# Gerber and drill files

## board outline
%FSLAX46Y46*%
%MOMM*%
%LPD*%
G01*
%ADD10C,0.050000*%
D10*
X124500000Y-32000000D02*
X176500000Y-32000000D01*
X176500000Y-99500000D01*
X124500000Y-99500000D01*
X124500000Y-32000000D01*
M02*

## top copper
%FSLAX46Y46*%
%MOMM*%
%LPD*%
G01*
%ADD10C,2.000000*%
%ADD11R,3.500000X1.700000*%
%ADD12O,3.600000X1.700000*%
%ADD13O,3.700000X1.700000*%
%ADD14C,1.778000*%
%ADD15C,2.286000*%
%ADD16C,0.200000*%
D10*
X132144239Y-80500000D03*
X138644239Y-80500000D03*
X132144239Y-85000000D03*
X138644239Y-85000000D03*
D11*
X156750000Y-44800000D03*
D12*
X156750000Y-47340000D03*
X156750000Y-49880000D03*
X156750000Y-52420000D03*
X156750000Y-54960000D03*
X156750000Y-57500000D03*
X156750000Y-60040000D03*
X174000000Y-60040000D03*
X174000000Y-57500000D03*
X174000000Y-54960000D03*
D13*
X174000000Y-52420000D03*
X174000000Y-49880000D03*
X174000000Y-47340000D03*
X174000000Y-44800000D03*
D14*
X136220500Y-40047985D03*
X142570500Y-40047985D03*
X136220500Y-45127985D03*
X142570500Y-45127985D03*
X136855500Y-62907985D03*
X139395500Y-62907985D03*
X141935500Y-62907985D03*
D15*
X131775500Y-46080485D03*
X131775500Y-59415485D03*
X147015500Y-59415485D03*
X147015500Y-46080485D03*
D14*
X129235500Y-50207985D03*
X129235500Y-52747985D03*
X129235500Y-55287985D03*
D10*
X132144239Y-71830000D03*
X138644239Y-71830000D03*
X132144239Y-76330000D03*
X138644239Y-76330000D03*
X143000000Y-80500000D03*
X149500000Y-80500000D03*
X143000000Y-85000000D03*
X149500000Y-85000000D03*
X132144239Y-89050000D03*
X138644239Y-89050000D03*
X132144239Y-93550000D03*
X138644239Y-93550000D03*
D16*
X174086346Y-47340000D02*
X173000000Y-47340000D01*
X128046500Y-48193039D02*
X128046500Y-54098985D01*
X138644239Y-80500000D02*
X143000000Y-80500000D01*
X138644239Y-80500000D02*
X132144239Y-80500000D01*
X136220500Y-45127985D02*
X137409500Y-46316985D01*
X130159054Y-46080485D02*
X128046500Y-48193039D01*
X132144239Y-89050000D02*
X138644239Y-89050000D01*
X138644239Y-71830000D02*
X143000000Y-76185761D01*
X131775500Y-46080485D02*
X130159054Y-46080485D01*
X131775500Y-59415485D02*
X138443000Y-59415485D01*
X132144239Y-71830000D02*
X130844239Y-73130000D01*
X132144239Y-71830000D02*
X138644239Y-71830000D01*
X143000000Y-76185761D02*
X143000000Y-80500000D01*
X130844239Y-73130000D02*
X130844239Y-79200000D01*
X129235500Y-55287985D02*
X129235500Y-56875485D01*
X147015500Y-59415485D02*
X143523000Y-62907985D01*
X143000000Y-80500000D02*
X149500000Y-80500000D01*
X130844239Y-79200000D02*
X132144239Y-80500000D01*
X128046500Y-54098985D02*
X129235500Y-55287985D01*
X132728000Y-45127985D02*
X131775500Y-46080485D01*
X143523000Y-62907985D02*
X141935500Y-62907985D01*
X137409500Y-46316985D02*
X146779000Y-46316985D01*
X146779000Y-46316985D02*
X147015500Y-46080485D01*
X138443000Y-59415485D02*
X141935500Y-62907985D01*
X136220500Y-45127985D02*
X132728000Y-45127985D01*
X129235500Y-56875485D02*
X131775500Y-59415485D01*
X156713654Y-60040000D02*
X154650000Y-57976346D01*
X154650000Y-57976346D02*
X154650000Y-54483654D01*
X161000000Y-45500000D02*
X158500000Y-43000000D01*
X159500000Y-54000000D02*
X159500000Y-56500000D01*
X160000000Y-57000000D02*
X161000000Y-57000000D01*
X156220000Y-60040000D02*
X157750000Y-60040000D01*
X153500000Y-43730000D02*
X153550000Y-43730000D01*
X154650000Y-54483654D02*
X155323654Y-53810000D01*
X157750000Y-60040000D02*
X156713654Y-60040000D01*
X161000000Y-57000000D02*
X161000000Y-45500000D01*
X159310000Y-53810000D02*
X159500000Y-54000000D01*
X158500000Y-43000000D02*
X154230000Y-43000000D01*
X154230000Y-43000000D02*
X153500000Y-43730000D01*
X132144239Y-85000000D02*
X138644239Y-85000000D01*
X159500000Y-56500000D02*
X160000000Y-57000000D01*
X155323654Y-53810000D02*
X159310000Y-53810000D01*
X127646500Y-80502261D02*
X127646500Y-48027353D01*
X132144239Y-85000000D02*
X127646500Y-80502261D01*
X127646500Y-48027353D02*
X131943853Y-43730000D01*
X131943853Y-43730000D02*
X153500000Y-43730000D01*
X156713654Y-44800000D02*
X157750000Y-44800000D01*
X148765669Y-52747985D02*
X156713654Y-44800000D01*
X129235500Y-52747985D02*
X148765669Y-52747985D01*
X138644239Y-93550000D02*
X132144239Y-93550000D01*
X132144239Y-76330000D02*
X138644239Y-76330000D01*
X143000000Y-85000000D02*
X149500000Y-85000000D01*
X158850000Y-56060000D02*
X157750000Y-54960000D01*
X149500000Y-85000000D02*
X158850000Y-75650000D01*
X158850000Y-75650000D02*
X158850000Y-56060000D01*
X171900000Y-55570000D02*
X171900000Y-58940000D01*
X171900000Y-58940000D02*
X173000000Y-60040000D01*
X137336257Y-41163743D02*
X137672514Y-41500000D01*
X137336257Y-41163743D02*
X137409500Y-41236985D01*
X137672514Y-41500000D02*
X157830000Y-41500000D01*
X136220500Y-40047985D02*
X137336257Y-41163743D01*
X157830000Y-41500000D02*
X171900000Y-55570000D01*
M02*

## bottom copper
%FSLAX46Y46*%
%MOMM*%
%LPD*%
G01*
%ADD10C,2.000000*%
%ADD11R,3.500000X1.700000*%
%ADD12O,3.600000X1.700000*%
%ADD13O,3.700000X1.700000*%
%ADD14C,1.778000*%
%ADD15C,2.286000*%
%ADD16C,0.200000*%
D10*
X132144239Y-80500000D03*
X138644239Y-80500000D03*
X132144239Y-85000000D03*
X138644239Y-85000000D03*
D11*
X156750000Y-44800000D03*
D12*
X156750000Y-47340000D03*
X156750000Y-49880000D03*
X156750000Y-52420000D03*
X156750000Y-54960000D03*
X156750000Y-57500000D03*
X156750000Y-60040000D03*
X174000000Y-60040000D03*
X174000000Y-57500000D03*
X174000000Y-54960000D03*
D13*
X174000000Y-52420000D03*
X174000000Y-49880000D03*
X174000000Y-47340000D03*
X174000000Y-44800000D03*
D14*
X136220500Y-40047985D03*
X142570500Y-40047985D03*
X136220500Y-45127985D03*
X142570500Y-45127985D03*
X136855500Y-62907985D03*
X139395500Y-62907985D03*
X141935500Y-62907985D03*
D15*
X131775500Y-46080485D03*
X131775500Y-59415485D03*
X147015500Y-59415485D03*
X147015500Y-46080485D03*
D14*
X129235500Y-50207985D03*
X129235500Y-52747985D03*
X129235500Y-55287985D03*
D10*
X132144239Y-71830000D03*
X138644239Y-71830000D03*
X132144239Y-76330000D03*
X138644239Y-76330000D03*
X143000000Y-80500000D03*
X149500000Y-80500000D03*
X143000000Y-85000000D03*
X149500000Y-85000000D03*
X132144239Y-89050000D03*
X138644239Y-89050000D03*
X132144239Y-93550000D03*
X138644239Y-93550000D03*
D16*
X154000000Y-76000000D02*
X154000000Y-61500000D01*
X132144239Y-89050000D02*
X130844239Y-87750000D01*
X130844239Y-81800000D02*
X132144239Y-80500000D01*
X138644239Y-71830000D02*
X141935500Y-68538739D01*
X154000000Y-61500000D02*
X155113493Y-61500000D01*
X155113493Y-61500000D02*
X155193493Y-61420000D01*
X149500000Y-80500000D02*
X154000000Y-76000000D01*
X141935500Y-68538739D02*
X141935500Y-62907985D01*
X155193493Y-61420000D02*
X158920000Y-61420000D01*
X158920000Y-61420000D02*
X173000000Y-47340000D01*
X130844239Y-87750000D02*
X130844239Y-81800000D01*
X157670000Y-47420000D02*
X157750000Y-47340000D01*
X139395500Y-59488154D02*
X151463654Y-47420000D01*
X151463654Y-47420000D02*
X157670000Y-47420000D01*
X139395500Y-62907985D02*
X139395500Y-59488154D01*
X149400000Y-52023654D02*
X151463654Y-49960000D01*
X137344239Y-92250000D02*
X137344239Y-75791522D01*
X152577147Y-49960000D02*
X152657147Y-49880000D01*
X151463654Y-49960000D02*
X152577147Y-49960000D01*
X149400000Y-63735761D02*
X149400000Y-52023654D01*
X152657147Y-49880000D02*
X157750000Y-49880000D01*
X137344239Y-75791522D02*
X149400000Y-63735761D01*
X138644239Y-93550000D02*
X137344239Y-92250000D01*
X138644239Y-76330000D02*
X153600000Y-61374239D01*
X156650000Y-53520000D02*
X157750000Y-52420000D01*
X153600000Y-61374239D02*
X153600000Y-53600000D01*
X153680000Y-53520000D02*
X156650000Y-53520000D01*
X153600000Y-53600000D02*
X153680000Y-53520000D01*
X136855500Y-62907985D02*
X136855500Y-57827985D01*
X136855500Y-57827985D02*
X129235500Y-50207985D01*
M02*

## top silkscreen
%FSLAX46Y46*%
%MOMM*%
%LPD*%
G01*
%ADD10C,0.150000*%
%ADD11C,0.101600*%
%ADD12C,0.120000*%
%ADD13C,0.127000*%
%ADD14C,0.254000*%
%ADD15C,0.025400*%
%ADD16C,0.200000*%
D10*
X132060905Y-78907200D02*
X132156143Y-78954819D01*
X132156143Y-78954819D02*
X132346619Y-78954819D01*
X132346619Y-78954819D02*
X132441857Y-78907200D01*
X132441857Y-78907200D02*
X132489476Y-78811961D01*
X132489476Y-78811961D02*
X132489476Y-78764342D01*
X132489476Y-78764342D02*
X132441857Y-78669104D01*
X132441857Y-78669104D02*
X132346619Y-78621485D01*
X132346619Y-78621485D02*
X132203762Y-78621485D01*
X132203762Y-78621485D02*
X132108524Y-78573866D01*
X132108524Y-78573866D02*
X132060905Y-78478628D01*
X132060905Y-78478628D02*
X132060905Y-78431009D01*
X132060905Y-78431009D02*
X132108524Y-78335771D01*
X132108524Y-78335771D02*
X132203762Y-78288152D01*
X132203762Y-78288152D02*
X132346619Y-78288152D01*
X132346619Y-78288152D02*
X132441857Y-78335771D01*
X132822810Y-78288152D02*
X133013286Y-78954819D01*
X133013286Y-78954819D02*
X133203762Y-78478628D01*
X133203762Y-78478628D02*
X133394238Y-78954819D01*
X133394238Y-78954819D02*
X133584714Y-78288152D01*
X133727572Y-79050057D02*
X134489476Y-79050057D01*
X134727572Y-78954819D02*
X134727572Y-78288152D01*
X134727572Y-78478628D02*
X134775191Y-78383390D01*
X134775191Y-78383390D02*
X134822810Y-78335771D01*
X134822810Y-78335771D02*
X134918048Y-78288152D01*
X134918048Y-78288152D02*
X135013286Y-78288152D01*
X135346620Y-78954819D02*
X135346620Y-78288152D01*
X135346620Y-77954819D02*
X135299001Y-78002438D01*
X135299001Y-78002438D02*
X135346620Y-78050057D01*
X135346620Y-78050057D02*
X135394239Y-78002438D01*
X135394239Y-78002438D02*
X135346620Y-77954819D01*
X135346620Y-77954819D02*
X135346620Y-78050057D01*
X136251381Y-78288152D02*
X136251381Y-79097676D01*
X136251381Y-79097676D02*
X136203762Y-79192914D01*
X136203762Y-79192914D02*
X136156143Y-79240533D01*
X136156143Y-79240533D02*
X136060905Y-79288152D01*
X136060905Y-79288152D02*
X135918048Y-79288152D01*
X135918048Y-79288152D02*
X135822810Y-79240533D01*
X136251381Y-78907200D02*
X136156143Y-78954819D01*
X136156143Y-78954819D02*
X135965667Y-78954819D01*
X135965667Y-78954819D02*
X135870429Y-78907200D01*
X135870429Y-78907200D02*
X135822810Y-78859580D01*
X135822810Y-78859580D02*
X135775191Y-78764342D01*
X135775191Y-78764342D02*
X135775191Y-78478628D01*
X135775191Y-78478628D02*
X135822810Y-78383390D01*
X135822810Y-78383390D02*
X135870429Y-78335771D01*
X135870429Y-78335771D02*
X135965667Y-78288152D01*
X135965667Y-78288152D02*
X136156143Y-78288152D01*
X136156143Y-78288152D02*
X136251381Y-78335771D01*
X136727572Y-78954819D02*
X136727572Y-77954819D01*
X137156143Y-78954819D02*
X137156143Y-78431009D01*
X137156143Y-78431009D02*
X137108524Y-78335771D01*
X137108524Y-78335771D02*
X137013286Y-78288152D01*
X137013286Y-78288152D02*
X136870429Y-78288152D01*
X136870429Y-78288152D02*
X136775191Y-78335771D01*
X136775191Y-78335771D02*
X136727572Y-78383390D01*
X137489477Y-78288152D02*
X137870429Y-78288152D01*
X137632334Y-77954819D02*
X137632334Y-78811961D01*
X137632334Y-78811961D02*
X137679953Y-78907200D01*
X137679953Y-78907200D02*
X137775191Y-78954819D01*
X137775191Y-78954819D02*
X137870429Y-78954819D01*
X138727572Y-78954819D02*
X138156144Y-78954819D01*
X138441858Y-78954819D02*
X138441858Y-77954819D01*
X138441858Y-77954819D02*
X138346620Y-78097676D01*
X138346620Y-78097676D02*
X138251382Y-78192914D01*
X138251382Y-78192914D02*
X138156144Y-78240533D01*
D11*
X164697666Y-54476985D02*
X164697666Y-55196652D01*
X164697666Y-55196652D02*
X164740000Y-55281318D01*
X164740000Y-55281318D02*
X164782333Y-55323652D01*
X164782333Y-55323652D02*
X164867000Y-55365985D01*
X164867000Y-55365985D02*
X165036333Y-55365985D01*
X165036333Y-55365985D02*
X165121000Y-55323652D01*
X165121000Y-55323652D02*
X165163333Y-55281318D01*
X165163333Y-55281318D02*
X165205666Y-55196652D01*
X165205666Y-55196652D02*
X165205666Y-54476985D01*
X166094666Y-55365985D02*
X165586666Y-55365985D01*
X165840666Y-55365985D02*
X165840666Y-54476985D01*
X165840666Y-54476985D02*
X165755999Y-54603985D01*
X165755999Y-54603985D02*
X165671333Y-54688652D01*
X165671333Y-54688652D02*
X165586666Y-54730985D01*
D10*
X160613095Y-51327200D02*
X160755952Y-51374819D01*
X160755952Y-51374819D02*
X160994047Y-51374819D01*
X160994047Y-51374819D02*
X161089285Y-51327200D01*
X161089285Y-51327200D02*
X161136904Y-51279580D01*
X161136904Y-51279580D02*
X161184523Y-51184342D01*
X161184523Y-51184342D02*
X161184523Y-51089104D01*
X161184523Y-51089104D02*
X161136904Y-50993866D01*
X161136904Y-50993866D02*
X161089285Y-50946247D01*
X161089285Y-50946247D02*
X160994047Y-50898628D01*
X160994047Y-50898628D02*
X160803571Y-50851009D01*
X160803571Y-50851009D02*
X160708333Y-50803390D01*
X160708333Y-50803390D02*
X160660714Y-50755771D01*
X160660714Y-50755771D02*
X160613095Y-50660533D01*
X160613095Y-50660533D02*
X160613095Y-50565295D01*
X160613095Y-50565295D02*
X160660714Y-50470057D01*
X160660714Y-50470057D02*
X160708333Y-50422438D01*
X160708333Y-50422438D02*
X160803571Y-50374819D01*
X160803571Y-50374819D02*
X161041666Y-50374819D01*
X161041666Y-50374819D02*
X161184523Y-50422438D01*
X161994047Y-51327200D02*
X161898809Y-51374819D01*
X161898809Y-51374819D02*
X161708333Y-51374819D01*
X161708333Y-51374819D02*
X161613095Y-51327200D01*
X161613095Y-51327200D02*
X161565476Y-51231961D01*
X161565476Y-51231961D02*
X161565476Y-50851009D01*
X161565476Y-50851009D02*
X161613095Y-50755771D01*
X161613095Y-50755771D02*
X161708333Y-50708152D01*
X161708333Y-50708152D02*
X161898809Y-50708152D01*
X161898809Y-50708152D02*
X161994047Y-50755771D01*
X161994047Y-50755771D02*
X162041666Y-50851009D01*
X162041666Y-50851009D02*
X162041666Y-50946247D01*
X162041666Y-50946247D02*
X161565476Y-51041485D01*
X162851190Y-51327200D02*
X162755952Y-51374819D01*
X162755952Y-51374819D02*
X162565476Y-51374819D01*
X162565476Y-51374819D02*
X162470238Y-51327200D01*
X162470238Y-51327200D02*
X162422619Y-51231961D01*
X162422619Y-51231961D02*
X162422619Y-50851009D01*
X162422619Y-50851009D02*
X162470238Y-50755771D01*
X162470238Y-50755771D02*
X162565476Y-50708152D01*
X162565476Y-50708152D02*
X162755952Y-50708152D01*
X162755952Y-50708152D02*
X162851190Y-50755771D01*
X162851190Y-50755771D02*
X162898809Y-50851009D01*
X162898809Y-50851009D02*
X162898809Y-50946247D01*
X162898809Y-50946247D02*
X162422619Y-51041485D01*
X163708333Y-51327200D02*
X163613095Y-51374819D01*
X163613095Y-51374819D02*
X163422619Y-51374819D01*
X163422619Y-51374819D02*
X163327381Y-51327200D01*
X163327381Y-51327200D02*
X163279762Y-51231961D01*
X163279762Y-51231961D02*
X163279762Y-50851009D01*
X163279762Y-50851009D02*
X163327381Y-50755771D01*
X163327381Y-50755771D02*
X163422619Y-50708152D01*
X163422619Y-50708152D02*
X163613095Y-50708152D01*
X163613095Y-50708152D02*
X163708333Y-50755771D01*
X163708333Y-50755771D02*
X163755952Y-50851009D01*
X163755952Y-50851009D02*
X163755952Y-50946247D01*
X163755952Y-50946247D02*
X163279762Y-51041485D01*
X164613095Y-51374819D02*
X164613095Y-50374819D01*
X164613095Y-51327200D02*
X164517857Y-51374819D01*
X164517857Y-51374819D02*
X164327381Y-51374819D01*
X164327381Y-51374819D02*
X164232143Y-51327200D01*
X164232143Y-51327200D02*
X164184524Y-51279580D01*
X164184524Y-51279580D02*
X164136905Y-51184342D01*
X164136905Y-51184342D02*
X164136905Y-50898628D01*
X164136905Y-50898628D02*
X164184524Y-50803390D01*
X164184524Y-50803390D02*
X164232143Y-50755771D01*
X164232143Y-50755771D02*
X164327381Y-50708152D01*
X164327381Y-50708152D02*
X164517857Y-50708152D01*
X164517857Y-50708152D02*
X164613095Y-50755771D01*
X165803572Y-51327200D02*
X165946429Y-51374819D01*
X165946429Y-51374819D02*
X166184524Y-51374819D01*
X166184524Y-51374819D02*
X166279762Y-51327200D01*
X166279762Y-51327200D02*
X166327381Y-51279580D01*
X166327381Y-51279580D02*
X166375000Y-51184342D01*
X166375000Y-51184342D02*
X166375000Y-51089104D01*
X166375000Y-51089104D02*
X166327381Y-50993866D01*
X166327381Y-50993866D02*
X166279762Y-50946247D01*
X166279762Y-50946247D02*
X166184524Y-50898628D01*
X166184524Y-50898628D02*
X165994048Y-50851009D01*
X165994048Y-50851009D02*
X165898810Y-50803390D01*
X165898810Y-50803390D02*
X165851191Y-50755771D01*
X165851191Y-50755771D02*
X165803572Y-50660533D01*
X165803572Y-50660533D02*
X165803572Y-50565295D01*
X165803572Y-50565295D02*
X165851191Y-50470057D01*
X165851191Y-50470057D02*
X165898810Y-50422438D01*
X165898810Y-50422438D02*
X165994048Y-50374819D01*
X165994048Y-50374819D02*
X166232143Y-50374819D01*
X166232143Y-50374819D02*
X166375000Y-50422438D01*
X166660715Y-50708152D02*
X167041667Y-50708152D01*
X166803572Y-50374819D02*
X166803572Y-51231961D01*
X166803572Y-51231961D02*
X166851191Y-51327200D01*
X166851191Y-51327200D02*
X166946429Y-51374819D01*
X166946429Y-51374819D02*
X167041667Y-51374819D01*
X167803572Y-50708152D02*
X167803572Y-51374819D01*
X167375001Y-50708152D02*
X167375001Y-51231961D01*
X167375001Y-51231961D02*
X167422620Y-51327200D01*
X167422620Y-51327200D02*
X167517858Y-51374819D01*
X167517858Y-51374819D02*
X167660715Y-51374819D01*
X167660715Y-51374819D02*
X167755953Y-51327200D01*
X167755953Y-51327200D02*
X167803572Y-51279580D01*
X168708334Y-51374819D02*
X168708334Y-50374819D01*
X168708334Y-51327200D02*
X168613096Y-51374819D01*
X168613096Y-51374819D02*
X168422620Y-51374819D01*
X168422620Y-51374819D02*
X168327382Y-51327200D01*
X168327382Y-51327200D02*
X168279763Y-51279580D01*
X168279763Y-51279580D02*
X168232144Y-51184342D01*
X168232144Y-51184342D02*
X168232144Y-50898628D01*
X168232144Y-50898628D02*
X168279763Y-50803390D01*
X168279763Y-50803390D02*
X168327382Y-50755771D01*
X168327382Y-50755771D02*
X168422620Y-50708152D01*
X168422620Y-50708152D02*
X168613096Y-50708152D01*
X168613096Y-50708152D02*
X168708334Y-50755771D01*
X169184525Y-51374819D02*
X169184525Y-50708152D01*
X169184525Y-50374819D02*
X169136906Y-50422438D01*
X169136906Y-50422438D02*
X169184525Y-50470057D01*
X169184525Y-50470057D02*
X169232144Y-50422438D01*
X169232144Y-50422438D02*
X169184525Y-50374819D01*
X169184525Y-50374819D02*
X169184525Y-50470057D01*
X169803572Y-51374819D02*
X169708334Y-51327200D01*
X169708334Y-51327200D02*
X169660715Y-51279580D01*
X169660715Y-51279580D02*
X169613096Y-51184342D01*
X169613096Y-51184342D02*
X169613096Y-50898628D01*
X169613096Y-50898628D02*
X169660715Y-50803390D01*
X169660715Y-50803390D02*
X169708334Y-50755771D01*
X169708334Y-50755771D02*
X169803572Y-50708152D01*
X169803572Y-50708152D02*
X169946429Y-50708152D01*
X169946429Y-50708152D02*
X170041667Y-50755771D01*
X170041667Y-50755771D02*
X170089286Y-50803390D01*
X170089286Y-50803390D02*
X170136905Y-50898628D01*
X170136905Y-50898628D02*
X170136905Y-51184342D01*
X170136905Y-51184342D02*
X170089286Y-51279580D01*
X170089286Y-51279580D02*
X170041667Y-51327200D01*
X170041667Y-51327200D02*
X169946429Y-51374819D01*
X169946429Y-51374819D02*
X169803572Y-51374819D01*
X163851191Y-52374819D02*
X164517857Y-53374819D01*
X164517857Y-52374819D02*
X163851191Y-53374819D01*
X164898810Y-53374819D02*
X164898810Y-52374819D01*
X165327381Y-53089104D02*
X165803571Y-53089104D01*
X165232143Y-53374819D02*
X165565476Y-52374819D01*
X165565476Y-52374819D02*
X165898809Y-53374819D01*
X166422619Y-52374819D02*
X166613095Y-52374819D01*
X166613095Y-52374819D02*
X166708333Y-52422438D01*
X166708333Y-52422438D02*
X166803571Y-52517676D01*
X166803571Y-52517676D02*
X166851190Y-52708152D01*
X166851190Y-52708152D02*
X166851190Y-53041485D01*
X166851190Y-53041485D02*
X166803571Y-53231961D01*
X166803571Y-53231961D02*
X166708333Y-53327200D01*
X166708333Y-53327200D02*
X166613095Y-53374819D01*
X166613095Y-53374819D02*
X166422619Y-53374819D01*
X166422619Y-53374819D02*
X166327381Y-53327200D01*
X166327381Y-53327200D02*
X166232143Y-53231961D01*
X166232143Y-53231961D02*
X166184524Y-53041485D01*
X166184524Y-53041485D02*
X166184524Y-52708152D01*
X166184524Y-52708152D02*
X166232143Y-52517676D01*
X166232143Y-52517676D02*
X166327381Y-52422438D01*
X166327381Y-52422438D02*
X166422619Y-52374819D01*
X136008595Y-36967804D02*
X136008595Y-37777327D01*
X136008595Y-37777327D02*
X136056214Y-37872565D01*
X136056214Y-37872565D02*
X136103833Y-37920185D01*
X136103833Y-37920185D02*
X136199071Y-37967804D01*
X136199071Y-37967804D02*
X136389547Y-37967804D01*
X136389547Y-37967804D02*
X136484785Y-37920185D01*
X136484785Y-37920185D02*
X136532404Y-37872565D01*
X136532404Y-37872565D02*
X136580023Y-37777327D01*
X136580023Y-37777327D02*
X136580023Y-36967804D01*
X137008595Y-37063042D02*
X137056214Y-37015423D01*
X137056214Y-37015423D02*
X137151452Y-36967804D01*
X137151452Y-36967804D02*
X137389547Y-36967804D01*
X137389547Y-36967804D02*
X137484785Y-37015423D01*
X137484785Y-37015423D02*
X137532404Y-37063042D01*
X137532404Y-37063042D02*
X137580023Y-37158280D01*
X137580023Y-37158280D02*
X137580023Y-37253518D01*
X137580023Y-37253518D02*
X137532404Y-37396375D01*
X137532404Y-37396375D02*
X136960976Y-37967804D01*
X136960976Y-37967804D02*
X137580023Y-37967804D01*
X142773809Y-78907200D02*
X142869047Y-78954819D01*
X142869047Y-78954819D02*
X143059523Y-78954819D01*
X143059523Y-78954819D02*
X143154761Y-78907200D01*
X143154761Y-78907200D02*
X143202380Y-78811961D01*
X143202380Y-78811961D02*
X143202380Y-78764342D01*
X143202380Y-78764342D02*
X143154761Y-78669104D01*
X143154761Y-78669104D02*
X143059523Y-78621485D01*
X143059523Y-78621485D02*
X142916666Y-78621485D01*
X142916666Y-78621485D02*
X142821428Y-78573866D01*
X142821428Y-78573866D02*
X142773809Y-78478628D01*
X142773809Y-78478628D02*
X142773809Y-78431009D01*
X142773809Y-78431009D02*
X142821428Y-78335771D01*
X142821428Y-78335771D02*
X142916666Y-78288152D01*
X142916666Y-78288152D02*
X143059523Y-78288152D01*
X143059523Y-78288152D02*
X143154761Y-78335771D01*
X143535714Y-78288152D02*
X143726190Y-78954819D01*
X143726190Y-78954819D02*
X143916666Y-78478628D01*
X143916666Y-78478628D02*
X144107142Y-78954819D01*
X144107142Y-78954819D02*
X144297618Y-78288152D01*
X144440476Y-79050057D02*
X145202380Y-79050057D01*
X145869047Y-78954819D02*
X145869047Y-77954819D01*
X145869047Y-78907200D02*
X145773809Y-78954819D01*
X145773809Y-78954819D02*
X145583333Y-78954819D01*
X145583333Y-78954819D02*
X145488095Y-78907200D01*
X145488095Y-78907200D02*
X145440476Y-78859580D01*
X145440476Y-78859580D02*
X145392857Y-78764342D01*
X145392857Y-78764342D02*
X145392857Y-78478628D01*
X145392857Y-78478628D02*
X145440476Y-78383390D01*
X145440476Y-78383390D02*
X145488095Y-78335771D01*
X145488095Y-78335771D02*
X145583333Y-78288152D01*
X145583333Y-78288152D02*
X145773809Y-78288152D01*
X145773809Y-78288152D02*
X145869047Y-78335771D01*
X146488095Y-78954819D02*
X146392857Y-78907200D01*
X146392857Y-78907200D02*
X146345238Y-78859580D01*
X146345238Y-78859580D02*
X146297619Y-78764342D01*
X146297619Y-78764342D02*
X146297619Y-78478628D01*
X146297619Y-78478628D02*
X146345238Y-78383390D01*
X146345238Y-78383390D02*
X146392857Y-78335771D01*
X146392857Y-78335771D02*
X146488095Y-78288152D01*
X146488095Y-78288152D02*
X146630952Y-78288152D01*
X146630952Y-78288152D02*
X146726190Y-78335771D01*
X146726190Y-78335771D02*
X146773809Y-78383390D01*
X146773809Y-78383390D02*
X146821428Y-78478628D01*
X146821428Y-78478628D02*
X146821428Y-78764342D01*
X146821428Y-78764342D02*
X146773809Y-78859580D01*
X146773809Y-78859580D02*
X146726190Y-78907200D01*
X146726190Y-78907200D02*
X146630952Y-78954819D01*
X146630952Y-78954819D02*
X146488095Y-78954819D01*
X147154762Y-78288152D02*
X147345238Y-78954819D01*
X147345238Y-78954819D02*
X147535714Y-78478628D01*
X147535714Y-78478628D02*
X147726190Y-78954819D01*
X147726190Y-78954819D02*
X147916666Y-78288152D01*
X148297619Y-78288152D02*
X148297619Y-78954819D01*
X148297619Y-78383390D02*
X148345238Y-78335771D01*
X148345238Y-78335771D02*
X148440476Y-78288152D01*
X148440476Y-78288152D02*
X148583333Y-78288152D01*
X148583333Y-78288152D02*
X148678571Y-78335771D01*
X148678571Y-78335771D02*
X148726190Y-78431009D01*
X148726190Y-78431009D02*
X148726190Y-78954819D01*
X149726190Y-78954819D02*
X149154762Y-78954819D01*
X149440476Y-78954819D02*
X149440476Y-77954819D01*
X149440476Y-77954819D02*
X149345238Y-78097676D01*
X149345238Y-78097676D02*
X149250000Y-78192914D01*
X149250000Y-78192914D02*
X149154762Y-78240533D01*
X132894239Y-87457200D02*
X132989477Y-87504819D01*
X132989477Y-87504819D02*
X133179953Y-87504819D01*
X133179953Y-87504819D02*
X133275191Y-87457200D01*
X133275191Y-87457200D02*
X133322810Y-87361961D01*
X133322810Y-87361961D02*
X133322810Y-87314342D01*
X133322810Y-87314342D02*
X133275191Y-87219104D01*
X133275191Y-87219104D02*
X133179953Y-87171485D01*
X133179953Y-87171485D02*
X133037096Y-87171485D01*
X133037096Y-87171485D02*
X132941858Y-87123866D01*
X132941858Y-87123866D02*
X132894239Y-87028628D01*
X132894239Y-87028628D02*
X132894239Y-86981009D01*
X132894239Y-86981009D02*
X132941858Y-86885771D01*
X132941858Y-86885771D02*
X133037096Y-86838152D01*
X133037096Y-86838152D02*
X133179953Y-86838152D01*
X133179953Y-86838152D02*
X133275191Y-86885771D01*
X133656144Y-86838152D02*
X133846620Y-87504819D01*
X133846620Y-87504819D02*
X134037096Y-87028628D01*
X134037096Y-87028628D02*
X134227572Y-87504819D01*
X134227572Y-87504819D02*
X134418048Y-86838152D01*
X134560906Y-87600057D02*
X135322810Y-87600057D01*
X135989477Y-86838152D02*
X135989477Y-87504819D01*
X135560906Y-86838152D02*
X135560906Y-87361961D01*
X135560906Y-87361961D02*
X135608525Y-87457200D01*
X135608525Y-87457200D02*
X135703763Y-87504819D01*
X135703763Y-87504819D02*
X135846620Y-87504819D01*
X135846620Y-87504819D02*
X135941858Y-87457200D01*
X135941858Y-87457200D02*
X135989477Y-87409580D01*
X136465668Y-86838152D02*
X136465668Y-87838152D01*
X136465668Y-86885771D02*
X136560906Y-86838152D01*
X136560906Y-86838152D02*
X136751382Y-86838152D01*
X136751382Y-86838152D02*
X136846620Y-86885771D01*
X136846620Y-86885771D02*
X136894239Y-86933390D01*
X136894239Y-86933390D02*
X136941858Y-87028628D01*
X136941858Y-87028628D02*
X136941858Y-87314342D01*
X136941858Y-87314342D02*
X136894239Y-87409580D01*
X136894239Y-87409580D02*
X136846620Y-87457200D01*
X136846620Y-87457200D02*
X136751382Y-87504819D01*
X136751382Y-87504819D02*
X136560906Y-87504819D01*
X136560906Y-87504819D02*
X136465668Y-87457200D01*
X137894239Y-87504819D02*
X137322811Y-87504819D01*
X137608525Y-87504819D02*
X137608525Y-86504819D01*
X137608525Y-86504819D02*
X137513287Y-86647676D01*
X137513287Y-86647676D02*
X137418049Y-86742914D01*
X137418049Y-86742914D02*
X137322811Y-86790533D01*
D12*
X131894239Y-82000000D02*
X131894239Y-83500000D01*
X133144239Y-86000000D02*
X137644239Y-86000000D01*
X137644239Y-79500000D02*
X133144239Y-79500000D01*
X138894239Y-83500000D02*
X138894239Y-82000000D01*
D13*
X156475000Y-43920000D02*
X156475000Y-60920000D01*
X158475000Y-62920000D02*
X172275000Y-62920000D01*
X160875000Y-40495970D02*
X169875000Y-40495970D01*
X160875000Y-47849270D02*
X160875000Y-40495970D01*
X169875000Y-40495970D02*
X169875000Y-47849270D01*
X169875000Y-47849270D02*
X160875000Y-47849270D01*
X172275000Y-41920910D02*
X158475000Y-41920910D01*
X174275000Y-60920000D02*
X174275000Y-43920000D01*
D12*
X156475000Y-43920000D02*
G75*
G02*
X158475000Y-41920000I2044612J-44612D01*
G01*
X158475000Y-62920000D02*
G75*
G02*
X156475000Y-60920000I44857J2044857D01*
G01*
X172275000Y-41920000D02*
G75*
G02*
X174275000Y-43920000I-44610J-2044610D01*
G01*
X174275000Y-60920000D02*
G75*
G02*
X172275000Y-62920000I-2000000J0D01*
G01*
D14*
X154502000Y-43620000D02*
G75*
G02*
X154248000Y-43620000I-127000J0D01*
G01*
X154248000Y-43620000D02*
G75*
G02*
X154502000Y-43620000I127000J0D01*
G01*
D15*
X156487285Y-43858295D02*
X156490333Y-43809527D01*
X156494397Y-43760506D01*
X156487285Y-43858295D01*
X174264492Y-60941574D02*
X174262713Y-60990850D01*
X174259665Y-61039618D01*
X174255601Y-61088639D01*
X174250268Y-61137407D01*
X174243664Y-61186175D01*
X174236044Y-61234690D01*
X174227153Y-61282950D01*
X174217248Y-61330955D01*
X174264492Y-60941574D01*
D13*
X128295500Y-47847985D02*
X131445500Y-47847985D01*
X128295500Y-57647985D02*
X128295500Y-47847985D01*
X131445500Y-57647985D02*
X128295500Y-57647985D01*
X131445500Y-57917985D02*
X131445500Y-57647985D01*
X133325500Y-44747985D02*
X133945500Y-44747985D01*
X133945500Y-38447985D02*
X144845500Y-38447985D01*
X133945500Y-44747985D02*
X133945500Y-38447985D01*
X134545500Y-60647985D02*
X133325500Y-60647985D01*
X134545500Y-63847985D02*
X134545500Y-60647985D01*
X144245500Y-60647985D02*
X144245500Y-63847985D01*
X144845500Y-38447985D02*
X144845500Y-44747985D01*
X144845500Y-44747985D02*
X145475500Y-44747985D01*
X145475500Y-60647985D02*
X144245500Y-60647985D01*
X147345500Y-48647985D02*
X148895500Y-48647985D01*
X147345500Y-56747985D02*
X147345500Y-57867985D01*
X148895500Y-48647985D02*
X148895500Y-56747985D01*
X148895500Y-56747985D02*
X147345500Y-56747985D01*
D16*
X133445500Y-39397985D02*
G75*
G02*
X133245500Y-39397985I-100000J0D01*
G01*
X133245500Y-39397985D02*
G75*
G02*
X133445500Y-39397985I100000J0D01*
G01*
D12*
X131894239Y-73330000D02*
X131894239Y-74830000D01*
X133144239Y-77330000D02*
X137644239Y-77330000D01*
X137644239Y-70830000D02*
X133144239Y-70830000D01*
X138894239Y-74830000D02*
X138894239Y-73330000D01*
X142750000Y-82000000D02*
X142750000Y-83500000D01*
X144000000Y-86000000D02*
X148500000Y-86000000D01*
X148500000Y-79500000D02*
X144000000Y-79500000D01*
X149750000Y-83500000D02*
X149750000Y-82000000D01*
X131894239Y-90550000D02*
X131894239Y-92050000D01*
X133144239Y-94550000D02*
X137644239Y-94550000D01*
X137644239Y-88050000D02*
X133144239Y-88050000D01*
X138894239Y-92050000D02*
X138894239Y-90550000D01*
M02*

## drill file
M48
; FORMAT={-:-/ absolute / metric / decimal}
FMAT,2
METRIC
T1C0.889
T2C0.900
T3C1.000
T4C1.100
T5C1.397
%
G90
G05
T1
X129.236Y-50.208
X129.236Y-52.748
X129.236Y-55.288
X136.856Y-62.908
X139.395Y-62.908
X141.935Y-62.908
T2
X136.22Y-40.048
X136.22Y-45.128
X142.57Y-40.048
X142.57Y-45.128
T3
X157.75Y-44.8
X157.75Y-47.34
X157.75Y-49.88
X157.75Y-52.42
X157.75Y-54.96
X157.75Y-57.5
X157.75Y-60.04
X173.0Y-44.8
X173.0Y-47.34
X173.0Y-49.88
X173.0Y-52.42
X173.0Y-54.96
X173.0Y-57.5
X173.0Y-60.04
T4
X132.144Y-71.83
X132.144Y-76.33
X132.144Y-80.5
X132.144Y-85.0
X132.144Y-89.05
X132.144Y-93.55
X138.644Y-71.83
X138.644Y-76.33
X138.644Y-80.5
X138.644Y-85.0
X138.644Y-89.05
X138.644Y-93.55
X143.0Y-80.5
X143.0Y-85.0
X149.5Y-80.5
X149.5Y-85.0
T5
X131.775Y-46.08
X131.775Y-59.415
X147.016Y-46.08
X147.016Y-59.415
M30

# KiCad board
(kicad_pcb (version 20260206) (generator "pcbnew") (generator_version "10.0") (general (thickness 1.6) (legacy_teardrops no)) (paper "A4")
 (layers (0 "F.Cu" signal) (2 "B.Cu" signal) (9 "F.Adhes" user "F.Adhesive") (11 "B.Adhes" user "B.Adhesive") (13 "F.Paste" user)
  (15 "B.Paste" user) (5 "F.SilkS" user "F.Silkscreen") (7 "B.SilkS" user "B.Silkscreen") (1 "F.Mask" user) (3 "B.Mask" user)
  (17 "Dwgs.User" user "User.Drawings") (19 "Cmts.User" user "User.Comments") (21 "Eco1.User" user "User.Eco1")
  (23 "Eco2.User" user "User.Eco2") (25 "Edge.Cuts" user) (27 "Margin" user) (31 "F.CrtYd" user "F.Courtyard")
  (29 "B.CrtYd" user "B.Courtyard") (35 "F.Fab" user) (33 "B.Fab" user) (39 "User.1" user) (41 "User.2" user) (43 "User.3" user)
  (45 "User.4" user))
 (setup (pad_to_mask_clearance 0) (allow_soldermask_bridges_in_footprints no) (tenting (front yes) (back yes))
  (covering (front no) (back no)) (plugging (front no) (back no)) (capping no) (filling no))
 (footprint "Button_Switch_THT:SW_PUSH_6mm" (layer "F.Cu") (at 132.144239 80.5)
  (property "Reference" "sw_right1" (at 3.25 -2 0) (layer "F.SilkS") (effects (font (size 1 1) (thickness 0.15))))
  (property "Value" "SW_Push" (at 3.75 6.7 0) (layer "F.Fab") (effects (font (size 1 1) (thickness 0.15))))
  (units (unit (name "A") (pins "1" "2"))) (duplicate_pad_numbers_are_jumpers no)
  (fp_line (start -0.25 1.5) (end -0.25 3) (stroke (width 0.12) (type solid)) (layer "F.SilkS"))
  (fp_line (start 1 5.5) (end 5.5 5.5) (stroke (width 0.12) (type solid)) (layer "F.SilkS"))
  (fp_line (start 5.5 -1) (end 1 -1) (stroke (width 0.12) (type solid)) (layer "F.SilkS"))
  (fp_line (start 6.75 3) (end 6.75 1.5) (stroke (width 0.12) (type solid)) (layer "F.SilkS"))
  (pad "1" thru_hole circle (at 0 0 90) (size 2 2) (drill 1.1) (layers "*.Cu" "*.Mask") (remove_unused_layers no) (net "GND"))
  (pad "1" thru_hole circle (at 6.5 0 90) (size 2 2) (drill 1.1) (layers "*.Cu" "*.Mask") (remove_unused_layers no) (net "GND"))
  (pad "2" thru_hole circle (at 0 4.5 90) (size 2 2) (drill 1.1) (layers "*.Cu" "*.Mask") (remove_unused_layers no)
   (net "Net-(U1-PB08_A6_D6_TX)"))
  (pad "2" thru_hole circle (at 6.5 4.5 90) (size 2 2) (drill 1.1) (layers "*.Cu" "*.Mask") (remove_unused_layers no)
   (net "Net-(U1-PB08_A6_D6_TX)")))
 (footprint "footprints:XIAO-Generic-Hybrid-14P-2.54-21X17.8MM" (layer "F.Cu") (at 165.375 52.42)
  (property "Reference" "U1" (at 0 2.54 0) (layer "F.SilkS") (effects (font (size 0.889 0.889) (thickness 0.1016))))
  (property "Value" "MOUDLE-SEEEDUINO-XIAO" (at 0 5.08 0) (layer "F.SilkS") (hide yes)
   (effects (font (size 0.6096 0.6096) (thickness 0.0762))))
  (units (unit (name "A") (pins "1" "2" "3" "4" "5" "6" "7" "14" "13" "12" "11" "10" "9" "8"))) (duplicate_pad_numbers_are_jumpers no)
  (fp_line (start -8.9 -8.5) (end -8.9 8.5) (stroke (width 0.127) (type solid)) (layer "F.SilkS"))
  (fp_line (start -6.9 10.5) (end 6.9 10.5) (stroke (width 0.127) (type solid)) (layer "F.SilkS"))
  (fp_line (start -4.5 -11.92403) (end 4.5 -11.92403) (stroke (width 0.127) (type solid)) (layer "F.SilkS"))
  (fp_line (start -4.5 -4.57073) (end -4.5 -11.92403) (stroke (width 0.127) (type solid)) (layer "F.SilkS"))
  (fp_line (start 4.5 -11.92403) (end 4.5 -4.57073) (stroke (width 0.127) (type solid)) (layer "F.SilkS"))
  (fp_line (start 4.5 -4.57073) (end -4.5 -4.57073) (stroke (width 0.127) (type solid)) (layer "F.SilkS"))
  (fp_line (start 6.9 -10.49909) (end -6.9 -10.49909) (stroke (width 0.127) (type solid)) (layer "F.SilkS"))
  (fp_line (start 8.9 8.5) (end 8.9 -8.5) (stroke (width 0.127) (type solid)) (layer "F.SilkS"))
  (fp_arc (start -8.9 -8.5) (mid -8.301491 -9.901491) (end -6.9 -10.5) (stroke (width 0.12) (type solid)) (layer "F.SilkS"))
  (fp_arc (start -6.9 10.5) (mid -8.301423 9.901423) (end -8.9 8.5) (stroke (width 0.12) (type solid)) (layer "F.SilkS"))
  (fp_arc (start 6.9 -10.5) (mid 8.301491 -9.901491) (end 8.9 -8.5) (stroke (width 0.12) (type solid)) (layer "F.SilkS"))
  (fp_arc (start 8.9 8.5) (mid 8.314214 9.914214) (end 6.9 10.5) (stroke (width 0.12) (type solid)) (layer "F.SilkS"))
  (fp_circle (center -11 -8.8) (end -11 -9.054) (stroke (width 0) (type solid)) (fill yes) (layer "F.SilkS"))
  (fp_poly
   (pts (xy -8.887715 -8.561705) (xy -8.884667 -8.610473) (xy -8.880603 -8.659494)) (stroke (width 0.0254) (type solid)) (fill no)
   (layer "F.SilkS"))
  (fp_poly
   (pts (xy 8.889492 8.521574) (xy 8.887713 8.57085) (xy 8.884665 8.619618) (xy 8.880601 8.668639) (xy 8.875268 8.717407)
    (xy 8.868664 8.766175) (xy 8.861044 8.81469) (xy 8.852153 8.86295) (xy 8.842248 8.910955))
   (stroke (width 0.0254) (type solid)) (fill no) (layer "F.SilkS"))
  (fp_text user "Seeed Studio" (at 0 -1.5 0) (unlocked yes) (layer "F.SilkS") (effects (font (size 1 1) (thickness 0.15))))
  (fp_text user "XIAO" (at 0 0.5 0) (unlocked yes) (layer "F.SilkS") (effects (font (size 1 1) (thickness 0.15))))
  (pad "1" thru_hole rect (at -7.625 -7.62) (size 3.5 1.7) (drill 1 (offset -1 0)) (layers "*.Cu" "*.Mask") (remove_unused_layers no)
   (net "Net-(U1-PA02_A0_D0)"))
  (pad "2" thru_hole oval (at -7.625 -5.08) (size 3.6 1.7) (drill 1 (offset -1 0)) (layers "*.Cu" "*.Mask") (remove_unused_layers no)
   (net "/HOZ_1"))
  (pad "3" thru_hole oval (at -7.625 -2.54) (size 3.6 1.7) (drill 1 (offset -1 0)) (layers "*.Cu" "*.Mask") (remove_unused_layers no)
   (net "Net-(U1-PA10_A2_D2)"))
  (pad "4" thru_hole oval (at -7.625 0) (size 3.6 1.7) (drill 1 (offset -1 0)) (layers "*.Cu" "*.Mask") (remove_unused_layers no)
   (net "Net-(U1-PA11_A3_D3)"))
  (pad "5" thru_hole oval (at -7.625 2.54) (size 3.6 1.7) (drill 1 (offset -1 0)) (layers "*.Cu" "*.Mask") (remove_unused_layers no)
   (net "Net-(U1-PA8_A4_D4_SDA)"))
  (pad "6" thru_hole oval (at -7.625 5.08 180) (size 3.6 1.7) (drill 1 (offset 1 0)) (layers "*.Cu" "*.Mask") (remove_unused_layers no)
   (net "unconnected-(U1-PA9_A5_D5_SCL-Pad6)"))
  (pad "7" thru_hole oval (at -7.625 7.62) (size 3.6 1.7) (drill 1 (offset -1 0)) (layers "*.Cu" "*.Mask") (remove_unused_layers no)
   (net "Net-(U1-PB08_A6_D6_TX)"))
  (pad "8" thru_hole oval (at 7.625 7.62) (size 3.6 1.7) (drill 1 (offset 1 0)) (layers "*.Cu" "*.Mask") (remove_unused_layers no)
   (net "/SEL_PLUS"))
  (pad "9" thru_hole oval (at 7.625 5.08) (size 3.6 1.7) (drill 1 (offset 1 0)) (layers "*.Cu" "*.Mask") (remove_unused_layers no)
   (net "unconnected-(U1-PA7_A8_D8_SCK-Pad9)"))
  (pad "10" thru_hole oval (at 7.625 2.54) (size 3.6 1.7) (drill 1 (offset 1 0)) (layers "*.Cu" "*.Mask") (remove_unused_layers no)
   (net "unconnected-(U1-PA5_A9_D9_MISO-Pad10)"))
  (pad "11" thru_hole oval (at 7.625 0) (size 3.7 1.7) (drill 1 (offset 1 0)) (layers "*.Cu" "*.Mask") (remove_unused_layers no)
   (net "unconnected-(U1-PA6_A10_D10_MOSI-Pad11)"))
  (pad "12" thru_hole oval (at 7.625 -2.54) (size 3.7 1.7) (drill 1 (offset 1 0)) (layers "*.Cu" "*.Mask") (remove_unused_layers no)
   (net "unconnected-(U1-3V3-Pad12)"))
  (pad "13" thru_hole oval (at 7.625 -5.08) (size 3.7 1.7) (drill 1 (offset 1 0)) (layers "*.Cu" "*.Mask") (remove_unused_layers no)
   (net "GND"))
  (pad "14" thru_hole oval (at 7.625 -7.62) (size 3.7 1.7) (drill 1 (offset 1 0)) (layers "*.Cu" "*.Mask") (remove_unused_layers no)
   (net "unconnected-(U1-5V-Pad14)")))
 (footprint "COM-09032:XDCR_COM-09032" (layer "F.Cu") (at 139.3955 52.747985)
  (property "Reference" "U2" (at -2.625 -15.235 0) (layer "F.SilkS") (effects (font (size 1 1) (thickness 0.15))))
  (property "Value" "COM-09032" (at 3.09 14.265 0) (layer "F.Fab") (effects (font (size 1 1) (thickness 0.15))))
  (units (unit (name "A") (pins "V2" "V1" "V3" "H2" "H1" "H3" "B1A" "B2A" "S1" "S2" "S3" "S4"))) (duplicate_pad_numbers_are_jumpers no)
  (fp_line (start -11.1 -4.9) (end -7.95 -4.9) (stroke (width 0.127) (type solid)) (layer "F.SilkS"))
  (fp_line (start -11.1 4.9) (end -11.1 -4.9) (stroke (width 0.127) (type solid)) (layer "F.SilkS"))
  (fp_line (start -7.95 4.9) (end -11.1 4.9) (stroke (width 0.127) (type solid)) (layer "F.SilkS"))
  (fp_line (start -7.95 5.17) (end -7.95 4.9) (stroke (width 0.127) (type solid)) (layer "F.SilkS"))
  (fp_line (start -6.07 -8) (end -5.45 -8) (stroke (width 0.127) (type solid)) (layer "F.SilkS"))
  (fp_line (start -5.45 -14.3) (end 5.45 -14.3) (stroke (width 0.127) (type solid)) (layer "F.SilkS"))
  (fp_line (start -5.45 -8) (end -5.45 -14.3) (stroke (width 0.127) (type solid)) (layer "F.SilkS"))
  (fp_line (start -4.85 7.9) (end -6.07 7.9) (stroke (width 0.127) (type solid)) (layer "F.SilkS"))
  (fp_line (start -4.85 11.1) (end -4.85 7.9) (stroke (width 0.127) (type solid)) (layer "F.SilkS"))
  (fp_line (start 4.85 7.9) (end 4.85 11.1) (stroke (width 0.127) (type solid)) (layer "F.SilkS"))
  (fp_line (start 5.45 -14.3) (end 5.45 -8) (stroke (width 0.127) (type solid)) (layer "F.SilkS"))
  (fp_line (start 5.45 -8) (end 6.08 -8) (stroke (width 0.127) (type solid)) (layer "F.SilkS"))
  (fp_line (start 6.08 7.9) (end 4.85 7.9) (stroke (width 0.127) (type solid)) (layer "F.SilkS"))
  (fp_line (start 7.95 -4.1) (end 9.5 -4.1) (stroke (width 0.127) (type solid)) (layer "F.SilkS"))
  (fp_line (start 7.95 4) (end 7.95 5.12) (stroke (width 0.127) (type solid)) (layer "F.SilkS"))
  (fp_line (start 9.5 -4.1) (end 9.5 4) (stroke (width 0.127) (type solid)) (layer "F.SilkS"))
  (fp_line (start 9.5 4) (end 7.95 4) (stroke (width 0.127) (type solid)) (layer "F.SilkS"))
  (fp_circle (center -6.05 -13.35) (end -5.95 -13.35) (stroke (width 0.2) (type solid)) (fill no) (layer "F.SilkS"))
  (pad "B1A" thru_hole circle (at -3.175 -12.7) (size 1.778 1.778) (drill 0.9) (layers "*.Cu" "*.Mask") (remove_unused_layers no)
   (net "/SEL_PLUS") (solder_mask_margin 0.102))
  (pad "B1B" thru_hole circle (at 3.175 -12.7) (size 1.778 1.778) (drill 0.9) (layers "*.Cu" "*.Mask") (remove_unused_layers no)
   (solder_mask_margin 0.102))
  (pad "B2A" thru_hole circle (at -3.175 -7.62) (size 1.778 1.778) (drill 0.9) (layers "*.Cu" "*.Mask") (remove_unused_layers no)
   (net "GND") (solder_mask_margin 0.102))
  (pad "B2B" thru_hole circle (at 3.175 -7.62) (size 1.778 1.778) (drill 0.9) (layers "*.Cu" "*.Mask") (remove_unused_layers no)
   (solder_mask_margin 0.102))
  (pad "H1" thru_hole circle (at -2.54 10.16) (size 1.778 1.778) (drill 0.889) (layers "*.Cu" "*.Mask") (remove_unused_layers no)
   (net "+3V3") (solder_mask_margin 0.102))
  (pad "H2" thru_hole circle (at 0 10.16) (size 1.778 1.778) (drill 0.889) (layers "*.Cu" "*.Mask") (remove_unused_layers no) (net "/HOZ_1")
   (solder_mask_margin 0.102))
  (pad "H3" thru_hole circle (at 2.54 10.16) (size 1.778 1.778) (drill 0.889) (layers "*.Cu" "*.Mask") (remove_unused_layers no) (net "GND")
   (solder_mask_margin 0.102))
  (pad "S1" thru_hole circle (at -7.62 -6.6675) (size 2.286 2.286) (drill 1.397) (layers "*.Cu" "*.Mask") (remove_unused_layers no)
   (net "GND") (solder_mask_margin 0.102))
  (pad "S2" thru_hole circle (at -7.62 6.6675) (size 2.286 2.286) (drill 1.397) (layers "*.Cu" "*.Mask") (remove_unused_layers no)
   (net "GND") (solder_mask_margin 0.102))
  (pad "S3" thru_hole circle (at 7.62 6.6675) (size 2.286 2.286) (drill 1.397) (layers "*.Cu" "*.Mask") (remove_unused_layers no)
   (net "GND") (solder_mask_margin 0.102))
  (pad "S4" thru_hole circle (at 7.62 -6.6675) (size 2.286 2.286) (drill 1.397) (layers "*.Cu" "*.Mask") (remove_unused_layers no)
   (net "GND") (solder_mask_margin 0.102))
  (pad "V1" thru_hole circle (at -10.16 -2.54) (size 1.778 1.778) (drill 0.889) (layers "*.Cu" "*.Mask") (remove_unused_layers no)
   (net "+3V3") (solder_mask_margin 0.102))
  (pad "V2" thru_hole circle (at -10.16 0) (size 1.778 1.778) (drill 0.889) (layers "*.Cu" "*.Mask") (remove_unused_layers no)
   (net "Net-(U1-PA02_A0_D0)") (solder_mask_margin 0.102))
  (pad "V3" thru_hole circle (at -10.16 2.54) (size 1.778 1.778) (drill 0.889) (layers "*.Cu" "*.Mask") (remove_unused_layers no)
   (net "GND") (solder_mask_margin 0.102)))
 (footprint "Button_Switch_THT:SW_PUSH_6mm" (layer "F.Cu") (at 132.144239 71.83)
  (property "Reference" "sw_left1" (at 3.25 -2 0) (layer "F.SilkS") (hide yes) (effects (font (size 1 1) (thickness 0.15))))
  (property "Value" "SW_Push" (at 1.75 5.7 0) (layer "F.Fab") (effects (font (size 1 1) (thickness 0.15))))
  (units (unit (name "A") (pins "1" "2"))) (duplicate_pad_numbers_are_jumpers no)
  (fp_line (start -0.25 1.5) (end -0.25 3) (stroke (width 0.12) (type solid)) (layer "F.SilkS"))
  (fp_line (start 1 5.5) (end 5.5 5.5) (stroke (width 0.12) (type solid)) (layer "F.SilkS"))
  (fp_line (start 5.5 -1) (end 1 -1) (stroke (width 0.12) (type solid)) (layer "F.SilkS"))
  (fp_line (start 6.75 3) (end 6.75 1.5) (stroke (width 0.12) (type solid)) (layer "F.SilkS"))
  (pad "1" thru_hole circle (at 0 0 90) (size 2 2) (drill 1.1) (layers "*.Cu" "*.Mask") (remove_unused_layers no) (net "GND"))
  (pad "1" thru_hole circle (at 6.5 0 90) (size 2 2) (drill 1.1) (layers "*.Cu" "*.Mask") (remove_unused_layers no) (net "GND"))
  (pad "2" thru_hole circle (at 0 4.5 90) (size 2 2) (drill 1.1) (layers "*.Cu" "*.Mask") (remove_unused_layers no)
   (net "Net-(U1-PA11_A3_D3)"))
  (pad "2" thru_hole circle (at 6.5 4.5 90) (size 2 2) (drill 1.1) (layers "*.Cu" "*.Mask") (remove_unused_layers no)
   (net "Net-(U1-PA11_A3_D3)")))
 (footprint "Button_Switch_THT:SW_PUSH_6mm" (layer "F.Cu") (at 143 80.5)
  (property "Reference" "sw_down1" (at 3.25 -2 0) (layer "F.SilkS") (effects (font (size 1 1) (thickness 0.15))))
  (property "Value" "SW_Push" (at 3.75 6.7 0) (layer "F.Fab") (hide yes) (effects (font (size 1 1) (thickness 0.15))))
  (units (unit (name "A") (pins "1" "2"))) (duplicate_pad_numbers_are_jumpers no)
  (fp_line (start -0.25 1.5) (end -0.25 3) (stroke (width 0.12) (type solid)) (layer "F.SilkS"))
  (fp_line (start 1 5.5) (end 5.5 5.5) (stroke (width 0.12) (type solid)) (layer "F.SilkS"))
  (fp_line (start 5.5 -1) (end 1 -1) (stroke (width 0.12) (type solid)) (layer "F.SilkS"))
  (fp_line (start 6.75 3) (end 6.75 1.5) (stroke (width 0.12) (type solid)) (layer "F.SilkS"))
  (pad "1" thru_hole circle (at 0 0 90) (size 2 2) (drill 1.1) (layers "*.Cu" "*.Mask") (remove_unused_layers no) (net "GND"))
  (pad "1" thru_hole circle (at 6.5 0 90) (size 2 2) (drill 1.1) (layers "*.Cu" "*.Mask") (remove_unused_layers no) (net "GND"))
  (pad "2" thru_hole circle (at 0 4.5 90) (size 2 2) (drill 1.1) (layers "*.Cu" "*.Mask") (remove_unused_layers no)
   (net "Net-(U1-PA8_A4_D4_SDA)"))
  (pad "2" thru_hole circle (at 6.5 4.5 90) (size 2 2) (drill 1.1) (layers "*.Cu" "*.Mask") (remove_unused_layers no)
   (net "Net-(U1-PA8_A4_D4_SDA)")))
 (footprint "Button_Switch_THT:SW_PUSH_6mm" (layer "F.Cu") (at 132.144239 89.05)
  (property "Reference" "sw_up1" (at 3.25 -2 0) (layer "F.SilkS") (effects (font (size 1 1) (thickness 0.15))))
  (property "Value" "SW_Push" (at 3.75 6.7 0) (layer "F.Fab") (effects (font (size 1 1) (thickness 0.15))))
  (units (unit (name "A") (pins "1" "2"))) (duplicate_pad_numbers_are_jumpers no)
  (fp_line (start -0.25 1.5) (end -0.25 3) (stroke (width 0.12) (type solid)) (layer "F.SilkS"))
  (fp_line (start 1 5.5) (end 5.5 5.5) (stroke (width 0.12) (type solid)) (layer "F.SilkS"))
  (fp_line (start 5.5 -1) (end 1 -1) (stroke (width 0.12) (type solid)) (layer "F.SilkS"))
  (fp_line (start 6.75 3) (end 6.75 1.5) (stroke (width 0.12) (type solid)) (layer "F.SilkS"))
  (pad "1" thru_hole circle (at 0 0 90) (size 2 2) (drill 1.1) (layers "*.Cu" "*.Mask") (remove_unused_layers no) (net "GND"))
  (pad "1" thru_hole circle (at 6.5 0 90) (size 2 2) (drill 1.1) (layers "*.Cu" "*.Mask") (remove_unused_layers no) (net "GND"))
  (pad "2" thru_hole circle (at 0 4.5 90) (size 2 2) (drill 1.1) (layers "*.Cu" "*.Mask") (remove_unused_layers no)
   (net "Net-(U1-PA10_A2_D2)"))
  (pad "2" thru_hole circle (at 6.5 4.5 90) (size 2 2) (drill 1.1) (layers "*.Cu" "*.Mask") (remove_unused_layers no)
   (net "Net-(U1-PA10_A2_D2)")))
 (gr_rect (start 124.5 32) (end 176.5 99.5) (stroke (width 0.05) (type default)) (fill no) (layer "Edge.Cuts"))
 (segment (start 174.086346 47.34) (end 173 47.34) (width 0.2) (layer "F.Cu") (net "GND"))
 (segment (start 128.0465 48.193039) (end 128.0465 54.098985) (width 0.2) (layer "F.Cu") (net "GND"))
 (segment (start 138.644239 80.5) (end 143 80.5) (width 0.2) (layer "F.Cu") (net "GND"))
 (segment (start 138.644239 80.5) (end 132.144239 80.5) (width 0.2) (layer "F.Cu") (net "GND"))
 (segment (start 136.2205 45.127985) (end 137.4095 46.316985) (width 0.2) (layer "F.Cu") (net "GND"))
 (segment (start 130.159054 46.080485) (end 128.0465 48.193039) (width 0.2) (layer "F.Cu") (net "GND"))
 (segment (start 132.144239 89.05) (end 138.644239 89.05) (width 0.2) (layer "F.Cu") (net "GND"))
 (segment (start 138.644239 71.83) (end 143 76.185761) (width 0.2) (layer "F.Cu") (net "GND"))
 (segment (start 131.7755 46.080485) (end 130.159054 46.080485) (width 0.2) (layer "F.Cu") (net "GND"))
 (segment (start 131.7755 59.415485) (end 138.443 59.415485) (width 0.2) (layer "F.Cu") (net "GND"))
 (segment (start 132.144239 71.83) (end 130.844239 73.13) (width 0.2) (layer "F.Cu") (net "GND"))
 (segment (start 132.144239 71.83) (end 138.644239 71.83) (width 0.2) (layer "F.Cu") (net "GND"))
 (segment (start 143 76.185761) (end 143 80.5) (width 0.2) (layer "F.Cu") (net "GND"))
 (segment (start 130.844239 73.13) (end 130.844239 79.2) (width 0.2) (layer "F.Cu") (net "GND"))
 (segment (start 129.2355 55.287985) (end 129.2355 56.875485) (width 0.2) (layer "F.Cu") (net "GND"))
 (segment (start 147.0155 59.415485) (end 143.523 62.907985) (width 0.2) (layer "F.Cu") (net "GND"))
 (segment (start 143 80.5) (end 149.5 80.5) (width 0.2) (layer "F.Cu") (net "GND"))
 (segment (start 130.844239 79.2) (end 132.144239 80.5) (width 0.2) (layer "F.Cu") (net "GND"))
 (segment (start 128.0465 54.098985) (end 129.2355 55.287985) (width 0.2) (layer "F.Cu") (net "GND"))
 (segment (start 132.728 45.127985) (end 131.7755 46.080485) (width 0.2) (layer "F.Cu") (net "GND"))
 (segment (start 143.523 62.907985) (end 141.9355 62.907985) (width 0.2) (layer "F.Cu") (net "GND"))
 (segment (start 137.4095 46.316985) (end 146.779 46.316985) (width 0.2) (layer "F.Cu") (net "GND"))
 (segment (start 146.779 46.316985) (end 147.0155 46.080485) (width 0.2) (layer "F.Cu") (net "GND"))
 (segment (start 138.443 59.415485) (end 141.9355 62.907985) (width 0.2) (layer "F.Cu") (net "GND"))
 (segment (start 136.2205 45.127985) (end 132.728 45.127985) (width 0.2) (layer "F.Cu") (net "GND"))
 (segment (start 129.2355 56.875485) (end 131.7755 59.415485) (width 0.2) (layer "F.Cu") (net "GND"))
 (segment (start 154 76) (end 154 61.5) (width 0.2) (layer "B.Cu") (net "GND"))
 (segment (start 132.144239 89.05) (end 130.844239 87.75) (width 0.2) (layer "B.Cu") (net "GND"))
 (segment (start 130.844239 81.8) (end 132.144239 80.5) (width 0.2) (layer "B.Cu") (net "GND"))
 (segment (start 138.644239 71.83) (end 141.9355 68.538739) (width 0.2) (layer "B.Cu") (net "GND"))
 (segment (start 154 61.5) (end 155.113493 61.5) (width 0.2) (layer "B.Cu") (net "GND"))
 (segment (start 155.113493 61.5) (end 155.193493 61.42) (width 0.2) (layer "B.Cu") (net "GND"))
 (segment (start 149.5 80.5) (end 154 76) (width 0.2) (layer "B.Cu") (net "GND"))
 (segment (start 141.9355 68.538739) (end 141.9355 62.907985) (width 0.2) (layer "B.Cu") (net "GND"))
 (segment (start 155.193493 61.42) (end 158.92 61.42) (width 0.2) (layer "B.Cu") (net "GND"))
 (segment (start 158.92 61.42) (end 173 47.34) (width 0.2) (layer "B.Cu") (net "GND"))
 (segment (start 130.844239 87.75) (end 130.844239 81.8) (width 0.2) (layer "B.Cu") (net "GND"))
 (segment (start 156.713654 60.04) (end 154.65 57.976346) (width 0.2) (layer "F.Cu") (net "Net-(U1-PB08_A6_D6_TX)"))
 (segment (start 154.65 57.976346) (end 154.65 54.483654) (width 0.2) (layer "F.Cu") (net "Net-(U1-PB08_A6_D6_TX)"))
 (segment (start 161 45.5) (end 158.5 43) (width 0.2) (layer "F.Cu") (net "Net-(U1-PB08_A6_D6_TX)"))
 (segment (start 159.5 54) (end 159.5 56.5) (width 0.2) (layer "F.Cu") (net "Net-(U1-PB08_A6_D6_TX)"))
 (segment (start 160 57) (end 161 57) (width 0.2) (layer "F.Cu") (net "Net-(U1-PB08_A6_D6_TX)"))
 (segment (start 156.22 60.04) (end 157.75 60.04) (width 0.2) (layer "F.Cu") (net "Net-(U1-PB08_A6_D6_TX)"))
 (segment (start 153.5 43.73) (end 153.55 43.73) (width 0.2) (layer "F.Cu") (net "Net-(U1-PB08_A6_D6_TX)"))
 (segment (start 154.65 54.483654) (end 155.323654 53.81) (width 0.2) (layer "F.Cu") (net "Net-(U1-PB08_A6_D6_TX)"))
 (segment (start 157.75 60.04) (end 156.713654 60.04) (width 0.2) (layer "F.Cu") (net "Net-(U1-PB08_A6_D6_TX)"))
 (segment (start 161 57) (end 161 45.5) (width 0.2) (layer "F.Cu") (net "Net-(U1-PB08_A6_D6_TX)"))
 (segment (start 159.31 53.81) (end 159.5 54) (width 0.2) (layer "F.Cu") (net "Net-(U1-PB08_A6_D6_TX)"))
 (segment (start 158.5 43) (end 154.23 43) (width 0.2) (layer "F.Cu") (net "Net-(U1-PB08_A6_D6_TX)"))
 (segment (start 154.23 43) (end 153.5 43.73) (width 0.2) (layer "F.Cu") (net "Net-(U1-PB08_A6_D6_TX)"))
 (segment (start 132.144239 85) (end 138.644239 85) (width 0.2) (layer "F.Cu") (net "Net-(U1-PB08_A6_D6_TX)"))
 (segment (start 159.5 56.5) (end 160 57) (width 0.2) (layer "F.Cu") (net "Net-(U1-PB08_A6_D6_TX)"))
 (segment (start 155.323654 53.81) (end 159.31 53.81) (width 0.2) (layer "F.Cu") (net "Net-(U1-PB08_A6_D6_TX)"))
 (segment (start 127.6465 80.502261) (end 127.6465 48.027353) (width 0.2) (layer "F.Cu") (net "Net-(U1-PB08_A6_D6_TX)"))
 (segment (start 132.144239 85) (end 127.6465 80.502261) (width 0.2) (layer "F.Cu") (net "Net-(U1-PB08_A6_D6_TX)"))
 (segment (start 127.6465 48.027353) (end 131.943853 43.73) (width 0.2) (layer "F.Cu") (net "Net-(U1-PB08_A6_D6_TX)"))
 (segment (start 131.943853 43.73) (end 153.5 43.73) (width 0.2) (layer "F.Cu") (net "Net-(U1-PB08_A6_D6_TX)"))
 (segment (start 156.713654 44.8) (end 157.75 44.8) (width 0.2) (layer "F.Cu") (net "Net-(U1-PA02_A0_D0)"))
 (segment (start 148.765669 52.747985) (end 156.713654 44.8) (width 0.2) (layer "F.Cu") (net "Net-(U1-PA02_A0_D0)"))
 (segment (start 129.2355 52.747985) (end 148.765669 52.747985) (width 0.2) (layer "F.Cu") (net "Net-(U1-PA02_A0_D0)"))
 (segment (start 157.67 47.42) (end 157.75 47.34) (width 0.2) (layer "B.Cu") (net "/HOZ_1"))
 (segment (start 139.3955 59.488154) (end 151.463654 47.42) (width 0.2) (layer "B.Cu") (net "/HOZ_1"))
 (segment (start 151.463654 47.42) (end 157.67 47.42) (width 0.2) (layer "B.Cu") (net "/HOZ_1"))
 (segment (start 139.3955 62.907985) (end 139.3955 59.488154) (width 0.2) (layer "B.Cu") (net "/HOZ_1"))
 (segment (start 138.644239 93.55) (end 132.144239 93.55) (width 0.2) (layer "F.Cu") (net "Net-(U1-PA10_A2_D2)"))
 (segment (start 149.4 52.023654) (end 151.463654 49.96) (width 0.2) (layer "B.Cu") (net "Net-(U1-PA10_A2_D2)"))
 (segment (start 137.344239 92.25) (end 137.344239 75.791522) (width 0.2) (layer "B.Cu") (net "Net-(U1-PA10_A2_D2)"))
 (segment (start 152.577147 49.96) (end 152.657147 49.88) (width 0.2) (layer "B.Cu") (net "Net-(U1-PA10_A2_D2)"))
 (segment (start 151.463654 49.96) (end 152.577147 49.96) (width 0.2) (layer "B.Cu") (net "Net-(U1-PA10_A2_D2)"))
 (segment (start 149.4 63.735761) (end 149.4 52.023654) (width 0.2) (layer "B.Cu") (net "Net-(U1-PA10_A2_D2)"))
 (segment (start 152.657147 49.88) (end 157.75 49.88) (width 0.2) (layer "B.Cu") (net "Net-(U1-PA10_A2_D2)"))
 (segment (start 137.344239 75.791522) (end 149.4 63.735761) (width 0.2) (layer "B.Cu") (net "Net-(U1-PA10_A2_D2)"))
 (segment (start 138.644239 93.55) (end 137.344239 92.25) (width 0.2) (layer "B.Cu") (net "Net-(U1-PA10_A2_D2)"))
 (segment (start 132.144239 76.33) (end 138.644239 76.33) (width 0.2) (layer "F.Cu") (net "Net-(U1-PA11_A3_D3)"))
 (segment (start 138.644239 76.33) (end 153.6 61.374239) (width 0.2) (layer "B.Cu") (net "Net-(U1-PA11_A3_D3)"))
 (segment (start 156.65 53.52) (end 157.75 52.42) (width 0.2) (layer "B.Cu") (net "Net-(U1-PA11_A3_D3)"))
 (segment (start 153.6 61.374239) (end 153.6 53.6) (width 0.2) (layer "B.Cu") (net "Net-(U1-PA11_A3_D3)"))
 (segment (start 153.68 53.52) (end 156.65 53.52) (width 0.2) (layer "B.Cu") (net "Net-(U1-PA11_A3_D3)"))
 (segment (start 153.6 53.6) (end 153.68 53.52) (width 0.2) (layer "B.Cu") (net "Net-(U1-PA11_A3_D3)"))
 (segment (start 143 85) (end 149.5 85) (width 0.2) (layer "F.Cu") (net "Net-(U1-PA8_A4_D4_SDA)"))
 (segment (start 158.85 56.06) (end 157.75 54.96) (width 0.2) (layer "F.Cu") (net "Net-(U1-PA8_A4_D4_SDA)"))
 (segment (start 149.5 85) (end 158.85 75.65) (width 0.2) (layer "F.Cu") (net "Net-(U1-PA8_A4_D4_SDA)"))
 (segment (start 158.85 75.65) (end 158.85 56.06) (width 0.2) (layer "F.Cu") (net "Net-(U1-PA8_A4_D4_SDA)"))
 (segment (start 171.9 55.57) (end 171.9 58.94) (width 0.2) (layer "F.Cu") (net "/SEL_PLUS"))
 (segment (start 171.9 58.94) (end 173 60.04) (width 0.2) (layer "F.Cu") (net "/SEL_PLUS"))
 (segment (start 137.336257 41.163743) (end 137.672514 41.5) (width 0.2) (layer "F.Cu") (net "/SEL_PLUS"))
 (segment (start 137.336257 41.163743) (end 137.4095 41.236985) (width 0.2) (layer "F.Cu") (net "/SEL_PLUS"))
 (segment (start 137.672514 41.5) (end 157.83 41.5) (width 0.2) (layer "F.Cu") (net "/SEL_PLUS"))
 (segment (start 136.2205 40.047985) (end 137.336257 41.163743) (width 0.2) (layer "F.Cu") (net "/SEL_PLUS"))
 (segment (start 157.83 41.5) (end 171.9 55.57) (width 0.2) (layer "F.Cu") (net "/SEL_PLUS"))
 (segment (start 136.8555 62.907985) (end 136.8555 57.827985) (width 0.2) (layer "B.Cu") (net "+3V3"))
 (segment (start 136.8555 57.827985) (end 129.2355 50.207985) (width 0.2) (layer "B.Cu") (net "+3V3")))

